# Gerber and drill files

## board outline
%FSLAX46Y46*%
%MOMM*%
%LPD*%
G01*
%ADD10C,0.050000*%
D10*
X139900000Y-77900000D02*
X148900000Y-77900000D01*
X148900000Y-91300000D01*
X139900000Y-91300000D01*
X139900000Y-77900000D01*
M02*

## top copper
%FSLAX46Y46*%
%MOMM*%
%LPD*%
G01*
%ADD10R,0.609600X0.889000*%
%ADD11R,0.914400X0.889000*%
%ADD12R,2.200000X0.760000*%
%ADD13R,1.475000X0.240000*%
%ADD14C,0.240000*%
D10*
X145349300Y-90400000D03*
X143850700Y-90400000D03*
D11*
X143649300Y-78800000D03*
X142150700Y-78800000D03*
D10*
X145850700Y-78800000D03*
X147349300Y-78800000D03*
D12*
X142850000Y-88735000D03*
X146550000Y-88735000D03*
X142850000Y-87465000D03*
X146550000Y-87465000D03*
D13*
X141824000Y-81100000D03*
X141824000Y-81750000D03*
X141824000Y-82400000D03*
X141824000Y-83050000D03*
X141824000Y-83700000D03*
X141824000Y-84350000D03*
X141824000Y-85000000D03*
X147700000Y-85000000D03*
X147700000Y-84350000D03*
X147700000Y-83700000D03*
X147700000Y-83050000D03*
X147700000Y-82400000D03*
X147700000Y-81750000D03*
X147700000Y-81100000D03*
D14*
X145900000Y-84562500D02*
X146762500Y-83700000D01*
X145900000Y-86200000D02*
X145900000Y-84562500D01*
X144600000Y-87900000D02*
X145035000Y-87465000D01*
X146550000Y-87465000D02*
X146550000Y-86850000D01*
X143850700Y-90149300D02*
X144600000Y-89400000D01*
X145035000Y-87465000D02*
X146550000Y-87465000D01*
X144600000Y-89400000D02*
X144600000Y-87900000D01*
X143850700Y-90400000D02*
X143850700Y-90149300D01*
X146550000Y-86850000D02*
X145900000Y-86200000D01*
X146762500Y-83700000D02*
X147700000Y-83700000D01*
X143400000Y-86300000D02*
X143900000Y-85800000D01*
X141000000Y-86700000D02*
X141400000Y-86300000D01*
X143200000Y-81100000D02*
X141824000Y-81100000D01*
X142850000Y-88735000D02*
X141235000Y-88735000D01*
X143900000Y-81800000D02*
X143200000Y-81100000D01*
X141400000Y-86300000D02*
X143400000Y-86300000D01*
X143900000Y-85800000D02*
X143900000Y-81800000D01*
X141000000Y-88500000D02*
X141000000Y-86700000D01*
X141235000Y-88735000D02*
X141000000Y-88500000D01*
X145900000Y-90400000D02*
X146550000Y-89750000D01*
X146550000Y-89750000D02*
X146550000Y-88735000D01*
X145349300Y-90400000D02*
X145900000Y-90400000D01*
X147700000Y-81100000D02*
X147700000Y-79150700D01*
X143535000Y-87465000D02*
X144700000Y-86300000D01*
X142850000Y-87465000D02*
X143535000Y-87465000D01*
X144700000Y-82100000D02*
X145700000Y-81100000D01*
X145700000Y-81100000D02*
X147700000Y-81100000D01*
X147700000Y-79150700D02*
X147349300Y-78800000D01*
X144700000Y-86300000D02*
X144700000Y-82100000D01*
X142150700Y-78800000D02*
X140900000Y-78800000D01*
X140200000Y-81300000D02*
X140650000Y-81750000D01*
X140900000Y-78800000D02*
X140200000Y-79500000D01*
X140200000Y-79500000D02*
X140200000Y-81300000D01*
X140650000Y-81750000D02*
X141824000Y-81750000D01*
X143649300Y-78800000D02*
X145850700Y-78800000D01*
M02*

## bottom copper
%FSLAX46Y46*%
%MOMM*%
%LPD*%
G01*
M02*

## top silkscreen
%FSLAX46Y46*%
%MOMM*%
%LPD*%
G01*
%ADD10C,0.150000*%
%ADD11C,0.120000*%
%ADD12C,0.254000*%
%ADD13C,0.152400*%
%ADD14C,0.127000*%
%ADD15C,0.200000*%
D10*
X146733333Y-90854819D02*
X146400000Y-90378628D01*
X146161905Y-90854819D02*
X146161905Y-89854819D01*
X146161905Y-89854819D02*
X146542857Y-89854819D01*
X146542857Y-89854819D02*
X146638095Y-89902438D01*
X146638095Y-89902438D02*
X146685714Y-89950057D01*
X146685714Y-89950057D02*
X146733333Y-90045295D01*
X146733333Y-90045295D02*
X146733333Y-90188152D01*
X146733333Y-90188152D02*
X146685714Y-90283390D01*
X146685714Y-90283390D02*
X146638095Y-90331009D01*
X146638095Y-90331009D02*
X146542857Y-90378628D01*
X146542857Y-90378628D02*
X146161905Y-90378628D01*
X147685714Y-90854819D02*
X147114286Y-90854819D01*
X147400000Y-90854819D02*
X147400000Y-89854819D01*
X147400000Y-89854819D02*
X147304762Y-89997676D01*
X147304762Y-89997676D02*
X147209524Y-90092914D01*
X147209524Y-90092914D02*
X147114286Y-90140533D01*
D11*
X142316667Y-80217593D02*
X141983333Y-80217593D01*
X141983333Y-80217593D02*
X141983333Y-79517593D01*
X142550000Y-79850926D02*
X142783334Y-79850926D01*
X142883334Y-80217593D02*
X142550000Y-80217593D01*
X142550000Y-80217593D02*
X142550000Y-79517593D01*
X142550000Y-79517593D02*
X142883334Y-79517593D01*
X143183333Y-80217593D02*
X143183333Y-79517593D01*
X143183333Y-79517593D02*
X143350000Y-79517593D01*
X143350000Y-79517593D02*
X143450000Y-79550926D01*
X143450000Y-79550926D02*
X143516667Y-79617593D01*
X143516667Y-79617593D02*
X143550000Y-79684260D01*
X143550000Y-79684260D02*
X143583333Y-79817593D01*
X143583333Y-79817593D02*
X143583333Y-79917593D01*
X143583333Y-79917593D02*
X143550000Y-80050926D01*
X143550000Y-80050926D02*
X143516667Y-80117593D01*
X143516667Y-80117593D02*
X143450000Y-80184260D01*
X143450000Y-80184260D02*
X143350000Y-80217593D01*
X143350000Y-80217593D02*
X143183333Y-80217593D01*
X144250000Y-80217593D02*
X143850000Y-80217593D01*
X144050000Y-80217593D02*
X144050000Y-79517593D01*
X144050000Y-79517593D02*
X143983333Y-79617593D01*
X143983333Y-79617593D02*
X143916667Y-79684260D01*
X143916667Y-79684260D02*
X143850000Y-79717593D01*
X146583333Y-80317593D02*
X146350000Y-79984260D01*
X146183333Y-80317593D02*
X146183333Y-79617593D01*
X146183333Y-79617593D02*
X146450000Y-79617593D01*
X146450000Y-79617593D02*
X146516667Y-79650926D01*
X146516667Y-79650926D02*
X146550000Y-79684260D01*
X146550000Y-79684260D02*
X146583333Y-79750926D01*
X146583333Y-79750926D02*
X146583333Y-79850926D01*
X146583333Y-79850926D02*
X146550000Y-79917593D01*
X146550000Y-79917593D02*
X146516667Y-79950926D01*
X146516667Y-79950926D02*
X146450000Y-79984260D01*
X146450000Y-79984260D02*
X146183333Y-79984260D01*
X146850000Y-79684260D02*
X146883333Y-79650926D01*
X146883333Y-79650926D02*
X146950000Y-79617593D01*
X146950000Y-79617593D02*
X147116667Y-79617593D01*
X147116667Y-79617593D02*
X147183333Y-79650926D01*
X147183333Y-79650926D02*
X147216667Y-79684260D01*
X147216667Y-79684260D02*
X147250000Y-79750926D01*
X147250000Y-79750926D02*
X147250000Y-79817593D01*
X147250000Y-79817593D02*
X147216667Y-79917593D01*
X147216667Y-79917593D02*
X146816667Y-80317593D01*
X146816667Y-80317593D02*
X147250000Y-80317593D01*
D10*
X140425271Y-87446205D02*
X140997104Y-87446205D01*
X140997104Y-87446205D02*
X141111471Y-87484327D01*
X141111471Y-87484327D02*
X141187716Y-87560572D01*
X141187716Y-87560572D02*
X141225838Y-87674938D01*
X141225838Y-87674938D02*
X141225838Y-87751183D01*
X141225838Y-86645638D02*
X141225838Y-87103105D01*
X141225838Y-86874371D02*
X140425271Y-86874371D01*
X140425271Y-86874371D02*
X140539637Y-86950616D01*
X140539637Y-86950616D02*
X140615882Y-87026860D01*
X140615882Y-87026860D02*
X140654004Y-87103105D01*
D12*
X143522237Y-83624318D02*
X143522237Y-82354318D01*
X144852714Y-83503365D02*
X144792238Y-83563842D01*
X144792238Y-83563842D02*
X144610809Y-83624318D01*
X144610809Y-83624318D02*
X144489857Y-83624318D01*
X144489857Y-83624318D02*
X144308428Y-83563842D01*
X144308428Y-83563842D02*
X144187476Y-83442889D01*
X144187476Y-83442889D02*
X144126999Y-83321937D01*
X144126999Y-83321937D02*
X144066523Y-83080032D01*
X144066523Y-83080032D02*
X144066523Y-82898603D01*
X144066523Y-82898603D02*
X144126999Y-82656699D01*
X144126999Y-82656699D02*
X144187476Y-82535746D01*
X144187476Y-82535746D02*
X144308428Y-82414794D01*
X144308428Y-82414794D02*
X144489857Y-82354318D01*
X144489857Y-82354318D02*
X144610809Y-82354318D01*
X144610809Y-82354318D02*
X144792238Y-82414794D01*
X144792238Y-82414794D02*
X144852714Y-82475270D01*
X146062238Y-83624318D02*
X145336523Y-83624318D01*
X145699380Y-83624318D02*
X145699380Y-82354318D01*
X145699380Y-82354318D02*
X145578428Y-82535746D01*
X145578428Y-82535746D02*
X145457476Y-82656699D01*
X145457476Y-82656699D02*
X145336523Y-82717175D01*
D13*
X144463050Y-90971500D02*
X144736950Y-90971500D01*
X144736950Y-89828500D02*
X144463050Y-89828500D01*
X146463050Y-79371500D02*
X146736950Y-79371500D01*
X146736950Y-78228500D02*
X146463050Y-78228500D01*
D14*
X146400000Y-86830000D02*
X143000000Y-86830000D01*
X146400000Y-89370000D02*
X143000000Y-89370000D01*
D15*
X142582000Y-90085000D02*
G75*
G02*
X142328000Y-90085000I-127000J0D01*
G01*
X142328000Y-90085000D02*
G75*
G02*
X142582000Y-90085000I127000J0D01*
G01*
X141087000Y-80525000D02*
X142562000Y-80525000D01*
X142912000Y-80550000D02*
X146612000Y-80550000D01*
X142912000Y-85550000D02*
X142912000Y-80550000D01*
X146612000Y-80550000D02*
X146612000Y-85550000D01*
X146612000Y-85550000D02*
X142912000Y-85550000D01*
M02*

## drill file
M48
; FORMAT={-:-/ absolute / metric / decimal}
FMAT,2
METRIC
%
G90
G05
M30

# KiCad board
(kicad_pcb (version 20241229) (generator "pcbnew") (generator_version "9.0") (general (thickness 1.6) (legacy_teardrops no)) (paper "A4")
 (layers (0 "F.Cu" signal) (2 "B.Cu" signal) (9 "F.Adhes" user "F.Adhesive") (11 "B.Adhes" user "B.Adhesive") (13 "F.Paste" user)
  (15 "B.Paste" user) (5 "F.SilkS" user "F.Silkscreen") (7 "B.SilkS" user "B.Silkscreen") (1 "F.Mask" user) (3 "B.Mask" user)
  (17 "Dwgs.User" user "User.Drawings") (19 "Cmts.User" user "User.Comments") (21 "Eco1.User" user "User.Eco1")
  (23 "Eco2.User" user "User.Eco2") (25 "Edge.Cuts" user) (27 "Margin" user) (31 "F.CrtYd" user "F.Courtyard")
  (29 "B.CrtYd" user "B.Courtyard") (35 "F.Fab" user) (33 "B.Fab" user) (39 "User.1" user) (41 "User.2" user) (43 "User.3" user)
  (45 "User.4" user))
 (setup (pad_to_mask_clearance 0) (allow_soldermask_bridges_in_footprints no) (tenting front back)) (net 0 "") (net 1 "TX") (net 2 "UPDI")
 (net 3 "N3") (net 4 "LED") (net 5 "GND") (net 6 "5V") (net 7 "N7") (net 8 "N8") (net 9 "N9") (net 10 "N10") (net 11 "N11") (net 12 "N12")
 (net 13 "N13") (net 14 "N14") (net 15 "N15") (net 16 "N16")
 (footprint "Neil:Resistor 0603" (layer "F.Cu") (at 144.6 90.4 180)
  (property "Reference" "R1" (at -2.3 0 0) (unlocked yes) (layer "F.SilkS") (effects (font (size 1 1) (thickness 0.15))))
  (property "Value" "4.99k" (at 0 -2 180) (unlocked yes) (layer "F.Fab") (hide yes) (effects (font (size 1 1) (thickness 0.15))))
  (fp_line (start 0.13695 -0.5715) (end -0.13695 -0.5715) (stroke (width 0.1524) (type solid)) (layer "F.SilkS"))
  (fp_line (start -0.13695 0.5715) (end 0.13695 0.5715) (stroke (width 0.1524) (type solid)) (layer "F.SilkS"))
  (pad "1" smd rect (at -0.7493 0 180) (size 0.6096 0.889) (layers "F.Cu" "F.Mask" "F.Paste") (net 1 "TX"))
  (pad "2" smd rect (at 0.7493 0 180) (size 0.6096 0.889) (layers "F.Cu" "F.Mask" "F.Paste") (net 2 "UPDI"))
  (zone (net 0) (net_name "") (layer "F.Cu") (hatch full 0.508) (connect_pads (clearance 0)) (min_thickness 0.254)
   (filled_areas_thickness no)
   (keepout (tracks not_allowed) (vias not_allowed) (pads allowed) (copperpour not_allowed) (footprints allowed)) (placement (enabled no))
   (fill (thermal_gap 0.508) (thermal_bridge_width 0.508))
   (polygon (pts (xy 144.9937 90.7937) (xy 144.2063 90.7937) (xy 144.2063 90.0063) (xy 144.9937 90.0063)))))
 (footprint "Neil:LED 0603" (layer "F.Cu") (at 142.9 78.8 180)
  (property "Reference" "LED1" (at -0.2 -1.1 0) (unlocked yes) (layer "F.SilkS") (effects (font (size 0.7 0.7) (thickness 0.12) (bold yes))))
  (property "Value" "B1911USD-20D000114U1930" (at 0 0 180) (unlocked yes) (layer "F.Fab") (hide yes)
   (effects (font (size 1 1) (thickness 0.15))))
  (pad "1" smd rect (at -0.7493 0 180) (size 0.9144 0.889) (layers "F.Cu" "F.Mask" "F.Paste") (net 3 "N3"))
  (pad "2" smd rect (at 0.7493 0 180) (size 0.9144 0.889) (layers "F.Cu" "F.Mask" "F.Paste") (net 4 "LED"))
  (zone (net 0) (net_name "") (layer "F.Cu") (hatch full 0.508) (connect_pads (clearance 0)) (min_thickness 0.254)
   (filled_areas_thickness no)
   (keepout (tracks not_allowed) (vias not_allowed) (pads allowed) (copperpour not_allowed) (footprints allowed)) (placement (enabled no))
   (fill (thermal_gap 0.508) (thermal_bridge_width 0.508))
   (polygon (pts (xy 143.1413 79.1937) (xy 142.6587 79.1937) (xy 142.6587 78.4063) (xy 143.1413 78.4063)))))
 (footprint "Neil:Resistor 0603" (layer "F.Cu") (at 146.6 78.8)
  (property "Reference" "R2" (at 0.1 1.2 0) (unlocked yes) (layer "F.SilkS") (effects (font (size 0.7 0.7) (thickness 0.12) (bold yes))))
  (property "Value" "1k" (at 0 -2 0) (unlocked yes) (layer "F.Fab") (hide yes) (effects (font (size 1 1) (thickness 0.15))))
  (fp_line (start -0.13695 0.5715) (end 0.13695 0.5715) (stroke (width 0.1524) (type solid)) (layer "F.SilkS"))
  (fp_line (start 0.13695 -0.5715) (end -0.13695 -0.5715) (stroke (width 0.1524) (type solid)) (layer "F.SilkS"))
  (pad "1" smd rect (at -0.7493 0) (size 0.6096 0.889) (layers "F.Cu" "F.Mask" "F.Paste") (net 3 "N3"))
  (pad "2" smd rect (at 0.7493 0) (size 0.6096 0.889) (layers "F.Cu" "F.Mask" "F.Paste") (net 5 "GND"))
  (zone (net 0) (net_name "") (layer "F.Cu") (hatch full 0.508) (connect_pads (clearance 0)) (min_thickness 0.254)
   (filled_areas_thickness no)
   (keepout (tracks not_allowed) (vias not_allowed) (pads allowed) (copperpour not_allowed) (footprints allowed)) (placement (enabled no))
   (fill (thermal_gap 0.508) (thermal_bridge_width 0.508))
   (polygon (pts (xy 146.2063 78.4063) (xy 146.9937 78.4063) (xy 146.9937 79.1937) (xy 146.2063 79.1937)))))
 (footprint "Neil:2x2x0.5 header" (layer "F.Cu") (at 144.7 88.1 90)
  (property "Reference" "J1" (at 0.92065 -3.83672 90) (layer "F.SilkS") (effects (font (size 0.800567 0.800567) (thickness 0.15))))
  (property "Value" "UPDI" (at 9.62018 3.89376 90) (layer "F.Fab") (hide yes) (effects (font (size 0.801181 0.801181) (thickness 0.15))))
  (fp_line (start 1.27 1.7) (end 1.27 -1.7) (stroke (width 0.127) (type solid)) (layer "F.SilkS"))
  (fp_line (start -1.27 1.7) (end -1.27 -1.7) (stroke (width 0.127) (type solid)) (layer "F.SilkS"))
  (fp_circle (center -1.985 -2.245) (end -1.858 -2.245) (stroke (width 0.2) (type solid)) (fill no) (layer "F.SilkS"))
  (pad "1" smd rect (at -0.635 -1.85 90) (size 0.76 2.2) (layers "F.Cu" "F.Mask" "F.Paste") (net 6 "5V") (solder_mask_margin 0.102))
  (pad "2" smd rect (at -0.635 1.85 90) (size 0.76 2.2) (layers "F.Cu" "F.Mask" "F.Paste") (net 1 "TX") (solder_mask_margin 0.102))
  (pad "3" smd rect (at 0.635 -1.85 90) (size 0.76 2.2) (layers "F.Cu" "F.Mask" "F.Paste") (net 5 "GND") (solder_mask_margin 0.102))
  (pad "4" smd rect (at 0.635 1.85 90) (size 0.76 2.2) (layers "F.Cu" "F.Mask" "F.Paste") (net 2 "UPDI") (solder_mask_margin 0.102)))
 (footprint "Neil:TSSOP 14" (layer "F.Cu") (at 144.762 83.05)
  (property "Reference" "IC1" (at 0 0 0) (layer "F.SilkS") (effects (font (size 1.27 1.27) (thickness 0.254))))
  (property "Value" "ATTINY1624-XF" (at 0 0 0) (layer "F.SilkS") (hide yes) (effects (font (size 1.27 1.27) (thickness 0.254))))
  (fp_line (start -3.675 -2.525) (end -2.2 -2.525) (stroke (width 0.2) (type solid)) (layer "F.SilkS"))
  (fp_line (start -1.85 -2.5) (end 1.85 -2.5) (stroke (width 0.2) (type solid)) (layer "F.SilkS"))
  (fp_line (start -1.85 2.5) (end -1.85 -2.5) (stroke (width 0.2) (type solid)) (layer "F.SilkS"))
  (fp_line (start 1.85 -2.5) (end 1.85 2.5) (stroke (width 0.2) (type solid)) (layer "F.SilkS"))
  (fp_line (start 1.85 2.5) (end -1.85 2.5) (stroke (width 0.2) (type solid)) (layer "F.SilkS"))
  (pad "1" smd rect (at -2.938 -1.95 90) (size 0.24 1.475) (layers "F.Cu" "F.Mask" "F.Paste") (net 6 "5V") (thermal_bridge_angle 45))
  (pad "2" smd rect (at -2.938 -1.3 90) (size 0.24 1.475) (layers "F.Cu" "F.Mask" "F.Paste") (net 4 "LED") (thermal_bridge_angle 45))
  (pad "3" smd rect (at -2.938 -0.65 90) (size 0.24 1.475) (layers "F.Cu" "F.Mask" "F.Paste") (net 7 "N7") (thermal_bridge_angle 45))
  (pad "4" smd rect (at -2.938 0 90) (size 0.24 1.475) (layers "F.Cu" "F.Mask" "F.Paste") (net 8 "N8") (thermal_bridge_angle 45))
  (pad "5" smd rect (at -2.938 0.65 90) (size 0.24 1.475) (layers "F.Cu" "F.Mask" "F.Paste") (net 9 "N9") (thermal_bridge_angle 45))
  (pad "6" smd rect (at -2.938 1.3 90) (size 0.24 1.475) (layers "F.Cu" "F.Mask" "F.Paste") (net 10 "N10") (thermal_bridge_angle 45))
  (pad "7" smd rect (at -2.938 1.95 90) (size 0.24 1.475) (layers "F.Cu" "F.Mask" "F.Paste") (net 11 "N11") (thermal_bridge_angle 45))
  (pad "8" smd rect (at 2.938 1.95 90) (size 0.24 1.475) (layers "F.Cu" "F.Mask" "F.Paste") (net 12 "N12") (thermal_bridge_angle 45))
  (pad "9" smd rect (at 2.938 1.3 90) (size 0.24 1.475) (layers "F.Cu" "F.Mask" "F.Paste") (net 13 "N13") (thermal_bridge_angle 45))
  (pad "10" smd rect (at 2.938 0.65 90) (size 0.24 1.475) (layers "F.Cu" "F.Mask" "F.Paste") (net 2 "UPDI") (thermal_bridge_angle 45))
  (pad "11" smd rect (at 2.938 0 90) (size 0.24 1.475) (layers "F.Cu" "F.Mask" "F.Paste") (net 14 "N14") (thermal_bridge_angle 45))
  (pad "12" smd rect (at 2.938 -0.65 90) (size 0.24 1.475) (layers "F.Cu" "F.Mask" "F.Paste") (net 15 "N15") (thermal_bridge_angle 45))
  (pad "13" smd rect (at 2.938 -1.3 90) (size 0.24 1.475) (layers "F.Cu" "F.Mask" "F.Paste") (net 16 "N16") (thermal_bridge_angle 45))
  (pad "14" smd rect (at 2.938 -1.95 90) (size 0.24 1.475) (layers "F.Cu" "F.Mask" "F.Paste") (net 5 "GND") (thermal_bridge_angle 45)))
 (gr_rect (start 139.9 77.9) (end 148.9 91.3) (stroke (width 0.05) (type default)) (fill no) (layer "Edge.Cuts"))
 (segment (start 145.9 84.5625) (end 146.7625 83.7) (width 0.24) (layer "F.Cu") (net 2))
 (segment (start 145.9 86.2) (end 145.9 84.5625) (width 0.24) (layer "F.Cu") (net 2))
 (segment (start 144.6 87.9) (end 145.035 87.465) (width 0.24) (layer "F.Cu") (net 2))
 (segment (start 146.55 87.465) (end 146.55 86.85) (width 0.24) (layer "F.Cu") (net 2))
 (segment (start 143.8507 90.1493) (end 144.6 89.4) (width 0.24) (layer "F.Cu") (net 2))
 (segment (start 145.035 87.465) (end 146.55 87.465) (width 0.24) (layer "F.Cu") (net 2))
 (segment (start 144.6 89.4) (end 144.6 87.9) (width 0.24) (layer "F.Cu") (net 2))
 (segment (start 143.8507 90.4) (end 143.8507 90.1493) (width 0.24) (layer "F.Cu") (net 2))
 (segment (start 146.55 86.85) (end 145.9 86.2) (width 0.24) (layer "F.Cu") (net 2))
 (segment (start 146.7625 83.7) (end 147.7 83.7) (width 0.24) (layer "F.Cu") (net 2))
 (segment (start 143.4 86.3) (end 143.9 85.8) (width 0.24) (layer "F.Cu") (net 6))
 (segment (start 141 86.7) (end 141.4 86.3) (width 0.24) (layer "F.Cu") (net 6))
 (segment (start 143.2 81.1) (end 141.824 81.1) (width 0.24) (layer "F.Cu") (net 6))
 (segment (start 142.85 88.735) (end 141.235 88.735) (width 0.24) (layer "F.Cu") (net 6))
 (segment (start 143.9 81.8) (end 143.2 81.1) (width 0.24) (layer "F.Cu") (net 6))
 (segment (start 141.4 86.3) (end 143.4 86.3) (width 0.24) (layer "F.Cu") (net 6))
 (segment (start 143.9 85.8) (end 143.9 81.8) (width 0.24) (layer "F.Cu") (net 6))
 (segment (start 141 88.5) (end 141 86.7) (width 0.24) (layer "F.Cu") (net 6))
 (segment (start 141.235 88.735) (end 141 88.5) (width 0.24) (layer "F.Cu") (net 6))
 (segment (start 145.9 90.4) (end 146.55 89.75) (width 0.24) (layer "F.Cu") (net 1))
 (segment (start 146.55 89.75) (end 146.55 88.735) (width 0.24) (layer "F.Cu") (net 1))
 (segment (start 145.3493 90.4) (end 145.9 90.4) (width 0.24) (layer "F.Cu") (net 1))
 (segment (start 147.7 81.1) (end 147.7 79.1507) (width 0.24) (layer "F.Cu") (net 5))
 (segment (start 143.535 87.465) (end 144.7 86.3) (width 0.24) (layer "F.Cu") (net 5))
 (segment (start 142.85 87.465) (end 143.535 87.465) (width 0.24) (layer "F.Cu") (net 5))
 (segment (start 144.7 82.1) (end 145.7 81.1) (width 0.24) (layer "F.Cu") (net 5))
 (segment (start 145.7 81.1) (end 147.7 81.1) (width 0.24) (layer "F.Cu") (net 5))
 (segment (start 147.7 79.1507) (end 147.3493 78.8) (width 0.24) (layer "F.Cu") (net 5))
 (segment (start 144.7 86.3) (end 144.7 82.1) (width 0.24) (layer "F.Cu") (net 5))
 (segment (start 142.1507 78.8) (end 140.9 78.8) (width 0.24) (layer "F.Cu") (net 4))
 (segment (start 140.2 81.3) (end 140.65 81.75) (width 0.24) (layer "F.Cu") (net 4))
 (segment (start 140.9 78.8) (end 140.2 79.5) (width 0.24) (layer "F.Cu") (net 4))
 (segment (start 140.2 79.5) (end 140.2 81.3) (width 0.24) (layer "F.Cu") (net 4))
 (segment (start 140.65 81.75) (end 141.824 81.75) (width 0.24) (layer "F.Cu") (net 4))
 (segment (start 143.6493 78.8) (end 145.8507 78.8) (width 0.24) (layer "F.Cu") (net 3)))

